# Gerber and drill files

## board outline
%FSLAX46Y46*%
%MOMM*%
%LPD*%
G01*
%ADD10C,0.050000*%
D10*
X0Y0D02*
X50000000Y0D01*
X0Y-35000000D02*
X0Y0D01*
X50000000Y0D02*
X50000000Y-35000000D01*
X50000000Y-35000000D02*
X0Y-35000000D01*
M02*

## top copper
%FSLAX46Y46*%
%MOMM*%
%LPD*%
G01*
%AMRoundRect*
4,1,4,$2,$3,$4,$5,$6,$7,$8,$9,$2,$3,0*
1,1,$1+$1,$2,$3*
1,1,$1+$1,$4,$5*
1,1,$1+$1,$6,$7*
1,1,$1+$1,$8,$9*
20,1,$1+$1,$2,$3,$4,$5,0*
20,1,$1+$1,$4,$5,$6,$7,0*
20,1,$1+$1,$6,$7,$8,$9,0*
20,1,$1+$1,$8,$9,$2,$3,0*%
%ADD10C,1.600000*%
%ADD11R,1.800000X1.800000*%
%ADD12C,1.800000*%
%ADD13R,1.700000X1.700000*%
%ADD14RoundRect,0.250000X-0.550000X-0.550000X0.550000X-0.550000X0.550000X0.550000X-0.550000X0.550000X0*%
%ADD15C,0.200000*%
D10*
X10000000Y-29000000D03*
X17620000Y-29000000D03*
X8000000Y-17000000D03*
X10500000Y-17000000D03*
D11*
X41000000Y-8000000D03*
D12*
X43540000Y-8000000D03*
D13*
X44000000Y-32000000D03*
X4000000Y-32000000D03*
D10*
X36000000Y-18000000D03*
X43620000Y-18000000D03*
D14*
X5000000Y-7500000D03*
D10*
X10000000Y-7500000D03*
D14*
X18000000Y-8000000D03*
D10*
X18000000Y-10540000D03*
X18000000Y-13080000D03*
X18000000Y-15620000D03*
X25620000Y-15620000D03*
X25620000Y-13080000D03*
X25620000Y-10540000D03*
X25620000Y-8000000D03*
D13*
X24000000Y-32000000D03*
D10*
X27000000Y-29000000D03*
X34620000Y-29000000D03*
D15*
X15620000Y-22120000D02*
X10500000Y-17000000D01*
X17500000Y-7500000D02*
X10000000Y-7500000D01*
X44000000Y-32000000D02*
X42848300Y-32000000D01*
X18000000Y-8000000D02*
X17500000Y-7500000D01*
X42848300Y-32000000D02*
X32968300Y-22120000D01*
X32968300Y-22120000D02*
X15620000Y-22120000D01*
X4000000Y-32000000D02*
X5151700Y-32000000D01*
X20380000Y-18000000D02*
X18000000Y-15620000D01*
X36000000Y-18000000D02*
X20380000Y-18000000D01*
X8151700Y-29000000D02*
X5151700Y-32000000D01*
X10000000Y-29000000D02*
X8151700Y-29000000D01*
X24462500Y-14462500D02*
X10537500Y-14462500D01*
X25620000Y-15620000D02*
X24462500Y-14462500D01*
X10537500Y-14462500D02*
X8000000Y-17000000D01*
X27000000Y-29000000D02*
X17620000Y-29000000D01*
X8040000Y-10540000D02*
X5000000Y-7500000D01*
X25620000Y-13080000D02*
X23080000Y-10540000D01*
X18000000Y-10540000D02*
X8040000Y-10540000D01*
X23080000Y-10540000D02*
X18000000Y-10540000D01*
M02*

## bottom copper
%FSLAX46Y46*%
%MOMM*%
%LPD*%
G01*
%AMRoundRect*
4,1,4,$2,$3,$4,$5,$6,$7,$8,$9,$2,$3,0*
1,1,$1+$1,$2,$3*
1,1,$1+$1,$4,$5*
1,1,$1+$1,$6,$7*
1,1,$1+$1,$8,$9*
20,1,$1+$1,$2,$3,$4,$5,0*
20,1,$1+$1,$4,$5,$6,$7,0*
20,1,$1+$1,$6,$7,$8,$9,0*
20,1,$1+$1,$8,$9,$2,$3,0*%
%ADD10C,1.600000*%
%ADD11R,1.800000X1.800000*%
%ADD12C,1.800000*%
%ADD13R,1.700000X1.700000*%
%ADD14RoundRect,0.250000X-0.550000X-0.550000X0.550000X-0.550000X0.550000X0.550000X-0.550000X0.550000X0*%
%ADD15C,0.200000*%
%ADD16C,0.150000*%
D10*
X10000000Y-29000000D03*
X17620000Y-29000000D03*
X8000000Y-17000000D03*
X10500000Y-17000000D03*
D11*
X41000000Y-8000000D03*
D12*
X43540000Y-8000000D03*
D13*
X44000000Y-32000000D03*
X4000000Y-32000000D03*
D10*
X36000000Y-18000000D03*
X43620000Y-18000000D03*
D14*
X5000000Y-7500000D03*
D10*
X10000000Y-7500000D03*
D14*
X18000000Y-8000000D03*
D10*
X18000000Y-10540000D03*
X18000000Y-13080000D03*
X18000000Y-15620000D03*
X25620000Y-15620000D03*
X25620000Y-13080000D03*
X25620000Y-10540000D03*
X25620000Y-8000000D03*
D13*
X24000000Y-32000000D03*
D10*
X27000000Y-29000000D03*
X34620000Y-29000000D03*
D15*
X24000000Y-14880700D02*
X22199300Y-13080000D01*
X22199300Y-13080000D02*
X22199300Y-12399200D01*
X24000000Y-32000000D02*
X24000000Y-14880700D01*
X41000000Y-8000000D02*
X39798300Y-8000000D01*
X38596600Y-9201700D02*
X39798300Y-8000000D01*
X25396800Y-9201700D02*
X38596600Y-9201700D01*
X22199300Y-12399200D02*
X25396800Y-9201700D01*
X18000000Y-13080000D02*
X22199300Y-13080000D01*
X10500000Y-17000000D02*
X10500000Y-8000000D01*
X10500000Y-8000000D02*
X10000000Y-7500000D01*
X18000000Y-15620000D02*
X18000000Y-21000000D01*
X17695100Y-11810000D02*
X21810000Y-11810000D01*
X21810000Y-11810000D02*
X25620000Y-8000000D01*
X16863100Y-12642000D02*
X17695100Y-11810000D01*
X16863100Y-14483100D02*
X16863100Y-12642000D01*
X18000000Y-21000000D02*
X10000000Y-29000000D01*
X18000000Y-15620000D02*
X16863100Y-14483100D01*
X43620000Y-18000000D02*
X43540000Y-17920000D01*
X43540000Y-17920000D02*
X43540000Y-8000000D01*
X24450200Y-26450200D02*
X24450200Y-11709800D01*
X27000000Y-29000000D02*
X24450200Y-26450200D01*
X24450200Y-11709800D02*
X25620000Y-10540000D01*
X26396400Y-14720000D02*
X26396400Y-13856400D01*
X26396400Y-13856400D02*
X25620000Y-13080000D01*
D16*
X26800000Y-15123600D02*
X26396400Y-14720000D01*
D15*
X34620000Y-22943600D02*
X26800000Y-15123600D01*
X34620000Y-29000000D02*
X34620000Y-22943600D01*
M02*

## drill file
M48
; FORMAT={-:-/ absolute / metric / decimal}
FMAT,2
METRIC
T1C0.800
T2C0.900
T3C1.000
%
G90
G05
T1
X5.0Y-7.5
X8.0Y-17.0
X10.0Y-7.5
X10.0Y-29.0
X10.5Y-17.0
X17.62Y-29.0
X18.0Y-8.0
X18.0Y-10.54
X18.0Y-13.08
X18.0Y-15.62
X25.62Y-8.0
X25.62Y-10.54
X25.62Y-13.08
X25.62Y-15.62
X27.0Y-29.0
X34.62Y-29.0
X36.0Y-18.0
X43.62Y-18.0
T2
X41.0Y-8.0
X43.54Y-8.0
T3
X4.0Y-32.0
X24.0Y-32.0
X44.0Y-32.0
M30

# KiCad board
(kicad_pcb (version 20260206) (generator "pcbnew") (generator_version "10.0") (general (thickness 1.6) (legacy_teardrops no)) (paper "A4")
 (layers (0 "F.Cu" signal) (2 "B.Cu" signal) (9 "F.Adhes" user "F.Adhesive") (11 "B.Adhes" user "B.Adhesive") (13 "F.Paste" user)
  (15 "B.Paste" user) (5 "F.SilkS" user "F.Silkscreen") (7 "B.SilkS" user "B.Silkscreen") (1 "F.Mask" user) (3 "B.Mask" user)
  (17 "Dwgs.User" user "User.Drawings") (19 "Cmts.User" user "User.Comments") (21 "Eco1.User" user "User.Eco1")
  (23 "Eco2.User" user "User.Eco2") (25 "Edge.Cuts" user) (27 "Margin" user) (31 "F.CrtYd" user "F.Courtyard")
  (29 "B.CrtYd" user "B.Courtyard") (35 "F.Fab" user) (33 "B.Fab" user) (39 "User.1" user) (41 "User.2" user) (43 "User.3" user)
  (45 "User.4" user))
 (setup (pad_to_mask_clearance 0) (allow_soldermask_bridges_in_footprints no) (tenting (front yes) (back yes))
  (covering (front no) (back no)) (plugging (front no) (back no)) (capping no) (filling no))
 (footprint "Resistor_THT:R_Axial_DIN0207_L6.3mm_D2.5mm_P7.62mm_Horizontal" (layer "F.Cu") (at 10 29)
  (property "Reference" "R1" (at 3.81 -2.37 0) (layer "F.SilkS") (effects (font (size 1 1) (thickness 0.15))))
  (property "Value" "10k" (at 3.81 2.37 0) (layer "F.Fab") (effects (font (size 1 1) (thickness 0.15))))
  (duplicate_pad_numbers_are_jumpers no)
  (pad "1" thru_hole circle (at 0 0) (size 1.6 1.6) (drill 0.8) (layers "*.Cu" "*.Mask") (remove_unused_layers no) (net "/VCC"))
  (pad "2" thru_hole circle (at 7.62 0) (size 1.6 1.6) (drill 0.8) (layers "*.Cu" "*.Mask") (remove_unused_layers no) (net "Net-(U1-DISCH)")))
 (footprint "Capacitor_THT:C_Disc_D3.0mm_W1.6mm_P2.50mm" (layer "F.Cu") (at 8 17)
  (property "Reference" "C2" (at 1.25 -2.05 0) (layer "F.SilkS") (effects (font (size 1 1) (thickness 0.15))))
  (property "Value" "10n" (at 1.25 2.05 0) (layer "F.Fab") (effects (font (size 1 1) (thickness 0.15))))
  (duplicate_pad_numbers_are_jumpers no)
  (pad "1" thru_hole circle (at 0 0) (size 1.6 1.6) (drill 0.8) (layers "*.Cu" "*.Mask") (remove_unused_layers no) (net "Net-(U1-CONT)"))
  (pad "2" thru_hole circle (at 2.5 0) (size 1.6 1.6) (drill 0.8) (layers "*.Cu" "*.Mask") (remove_unused_layers no) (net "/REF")))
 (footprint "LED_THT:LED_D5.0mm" (layer "F.Cu") (at 41 8)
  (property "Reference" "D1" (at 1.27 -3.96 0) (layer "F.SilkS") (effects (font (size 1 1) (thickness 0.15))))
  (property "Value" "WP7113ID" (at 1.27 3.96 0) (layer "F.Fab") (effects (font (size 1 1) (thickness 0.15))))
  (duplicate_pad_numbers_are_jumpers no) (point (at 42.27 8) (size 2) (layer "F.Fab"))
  (pad "1" thru_hole rect (at 0 0) (size 1.8 1.8) (drill 0.9) (layers "*.Cu" "*.Mask") (remove_unused_layers no) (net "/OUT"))
  (pad "2" thru_hole circle (at 2.54 0) (size 1.8 1.8) (drill 0.9) (layers "*.Cu" "*.Mask") (remove_unused_layers no) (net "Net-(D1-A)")))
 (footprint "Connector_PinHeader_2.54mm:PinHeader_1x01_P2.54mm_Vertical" (layer "F.Cu") (at 44 32)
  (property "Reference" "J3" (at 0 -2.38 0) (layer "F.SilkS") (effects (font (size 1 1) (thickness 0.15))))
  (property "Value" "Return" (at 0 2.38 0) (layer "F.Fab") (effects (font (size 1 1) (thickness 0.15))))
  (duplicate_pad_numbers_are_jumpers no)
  (pad "1" thru_hole rect (at 0 0) (size 1.7 1.7) (drill 1) (layers "*.Cu" "*.Mask") (remove_unused_layers no) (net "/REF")))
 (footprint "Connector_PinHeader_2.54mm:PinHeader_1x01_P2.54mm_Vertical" (layer "F.Cu") (at 4 32)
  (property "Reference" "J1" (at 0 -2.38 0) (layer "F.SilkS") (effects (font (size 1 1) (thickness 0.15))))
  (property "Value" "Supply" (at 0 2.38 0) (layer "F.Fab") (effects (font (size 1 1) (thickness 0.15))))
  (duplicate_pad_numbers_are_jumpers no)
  (pad "1" thru_hole rect (at 0 0) (size 1.7 1.7) (drill 1) (layers "*.Cu" "*.Mask") (remove_unused_layers no) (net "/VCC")))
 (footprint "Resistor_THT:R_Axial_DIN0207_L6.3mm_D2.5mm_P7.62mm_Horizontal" (layer "F.Cu") (at 36 18)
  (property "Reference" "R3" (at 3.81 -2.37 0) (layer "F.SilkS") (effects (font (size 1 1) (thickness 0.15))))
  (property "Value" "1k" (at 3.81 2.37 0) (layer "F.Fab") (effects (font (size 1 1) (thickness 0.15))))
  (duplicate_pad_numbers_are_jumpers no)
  (pad "1" thru_hole circle (at 0 0) (size 1.6 1.6) (drill 0.8) (layers "*.Cu" "*.Mask") (remove_unused_layers no) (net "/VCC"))
  (pad "2" thru_hole circle (at 7.62 0) (size 1.6 1.6) (drill 0.8) (layers "*.Cu" "*.Mask") (remove_unused_layers no) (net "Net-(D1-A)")))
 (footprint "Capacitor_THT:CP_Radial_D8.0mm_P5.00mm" (layer "F.Cu") (at 5 7.5)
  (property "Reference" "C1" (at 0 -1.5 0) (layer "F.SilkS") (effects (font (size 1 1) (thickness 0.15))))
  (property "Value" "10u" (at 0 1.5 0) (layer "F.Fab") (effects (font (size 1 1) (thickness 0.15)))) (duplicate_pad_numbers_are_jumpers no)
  (pad "1" thru_hole roundrect (at 0 0) (size 1.6 1.6) (drill 0.8) (layers "*.Cu" "*.Mask") (remove_unused_layers no)
   (roundrect_rratio 0.15625) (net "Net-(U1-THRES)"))
  (pad "2" thru_hole circle (at 5 0) (size 1.6 1.6) (drill 0.8) (layers "*.Cu" "*.Mask") (remove_unused_layers no) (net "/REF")))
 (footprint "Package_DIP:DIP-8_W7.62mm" (layer "F.Cu") (at 18 8)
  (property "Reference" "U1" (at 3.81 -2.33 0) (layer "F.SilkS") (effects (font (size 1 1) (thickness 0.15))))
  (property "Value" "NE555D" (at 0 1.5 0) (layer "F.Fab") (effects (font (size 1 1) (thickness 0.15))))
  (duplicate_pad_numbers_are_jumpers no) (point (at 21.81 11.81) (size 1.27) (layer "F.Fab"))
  (pad "1" thru_hole roundrect (at 0 0) (size 1.6 1.6) (drill 0.8) (layers "*.Cu" "*.Mask") (remove_unused_layers no)
   (roundrect_rratio 0.15625) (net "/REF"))
  (pad "2" thru_hole circle (at 0 2.54) (size 1.6 1.6) (drill 0.8) (layers "*.Cu" "*.Mask") (remove_unused_layers no) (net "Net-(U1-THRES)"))
  (pad "3" thru_hole circle (at 0 5.08) (size 1.6 1.6) (drill 0.8) (layers "*.Cu" "*.Mask") (remove_unused_layers no) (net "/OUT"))
  (pad "4" thru_hole circle (at 0 7.62) (size 1.6 1.6) (drill 0.8) (layers "*.Cu" "*.Mask") (remove_unused_layers no) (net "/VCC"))
  (pad "5" thru_hole circle (at 7.62 7.62) (size 1.6 1.6) (drill 0.8) (layers "*.Cu" "*.Mask") (remove_unused_layers no)
   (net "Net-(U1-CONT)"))
  (pad "6" thru_hole circle (at 7.62 5.08) (size 1.6 1.6) (drill 0.8) (layers "*.Cu" "*.Mask") (remove_unused_layers no)
   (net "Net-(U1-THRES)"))
  (pad "7" thru_hole circle (at 7.62 2.54) (size 1.6 1.6) (drill 0.8) (layers "*.Cu" "*.Mask") (remove_unused_layers no)
   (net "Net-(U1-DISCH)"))
  (pad "8" thru_hole circle (at 7.62 0) (size 1.6 1.6) (drill 0.8) (layers "*.Cu" "*.Mask") (remove_unused_layers no) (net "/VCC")))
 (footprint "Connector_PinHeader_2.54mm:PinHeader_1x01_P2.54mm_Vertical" (layer "F.Cu") (at 24 32)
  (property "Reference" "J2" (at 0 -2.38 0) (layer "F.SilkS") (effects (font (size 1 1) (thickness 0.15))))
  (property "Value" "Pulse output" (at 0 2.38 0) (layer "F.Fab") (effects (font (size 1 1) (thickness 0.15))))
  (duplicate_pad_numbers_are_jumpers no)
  (pad "1" thru_hole rect (at 0 0) (size 1.7 1.7) (drill 1) (layers "*.Cu" "*.Mask") (remove_unused_layers no) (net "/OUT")))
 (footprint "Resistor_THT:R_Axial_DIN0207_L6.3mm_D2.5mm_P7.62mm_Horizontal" (layer "F.Cu") (at 27 29)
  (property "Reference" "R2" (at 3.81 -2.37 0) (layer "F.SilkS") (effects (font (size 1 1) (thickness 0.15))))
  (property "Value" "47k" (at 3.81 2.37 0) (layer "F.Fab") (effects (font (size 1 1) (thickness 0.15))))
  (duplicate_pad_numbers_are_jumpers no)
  (pad "1" thru_hole circle (at 0 0) (size 1.6 1.6) (drill 0.8) (layers "*.Cu" "*.Mask") (remove_unused_layers no) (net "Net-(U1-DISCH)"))
  (pad "2" thru_hole circle (at 7.62 0) (size 1.6 1.6) (drill 0.8) (layers "*.Cu" "*.Mask") (remove_unused_layers no) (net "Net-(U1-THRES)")))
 (gr_line (start 0 0) (end 50 0) (stroke (width 0.05) (type default)) (layer "Edge.Cuts"))
 (gr_line (start 0 35) (end 0 0) (stroke (width 0.05) (type default)) (layer "Edge.Cuts"))
 (gr_line (start 50 0) (end 50 35) (stroke (width 0.05) (type default)) (layer "Edge.Cuts"))
 (gr_line (start 50 35) (end 0 35) (stroke (width 0.05) (type default)) (layer "Edge.Cuts"))
 (segment (start 24 14.8807) (end 22.1993 13.08) (width 0.2) (layer "B.Cu") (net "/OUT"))
 (segment (start 22.1993 13.08) (end 22.1993 12.3992) (width 0.2) (layer "B.Cu") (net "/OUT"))
 (segment (start 24 32) (end 24 14.8807) (width 0.2) (layer "B.Cu") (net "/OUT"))
 (segment (start 41 8) (end 39.7983 8) (width 0.2) (layer "B.Cu") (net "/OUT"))
 (segment (start 38.5966 9.2017) (end 39.7983 8) (width 0.2) (layer "B.Cu") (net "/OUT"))
 (segment (start 25.3968 9.2017) (end 38.5966 9.2017) (width 0.2) (layer "B.Cu") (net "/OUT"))
 (segment (start 22.1993 12.3992) (end 25.3968 9.2017) (width 0.2) (layer "B.Cu") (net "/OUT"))
 (segment (start 18 13.08) (end 22.1993 13.08) (width 0.2) (layer "B.Cu") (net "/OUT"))
 (segment (start 15.62 22.12) (end 10.5 17) (width 0.2) (layer "F.Cu") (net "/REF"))
 (segment (start 17.5 7.5) (end 10 7.5) (width 0.2) (layer "F.Cu") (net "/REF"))
 (segment (start 44 32) (end 42.8483 32) (width 0.2) (layer "F.Cu") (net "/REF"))
 (segment (start 18 8) (end 17.5 7.5) (width 0.2) (layer "F.Cu") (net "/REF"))
 (segment (start 42.8483 32) (end 32.9683 22.12) (width 0.2) (layer "F.Cu") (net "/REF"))
 (segment (start 32.9683 22.12) (end 15.62 22.12) (width 0.2) (layer "F.Cu") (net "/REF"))
 (segment (start 10.5 17) (end 10.5 8) (width 0.2) (layer "B.Cu") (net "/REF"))
 (segment (start 10.5 8) (end 10 7.5) (width 0.2) (layer "B.Cu") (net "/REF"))
 (segment (start 4 32) (end 5.1517 32) (width 0.2) (layer "F.Cu") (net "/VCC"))
 (segment (start 20.38 18) (end 18 15.62) (width 0.2) (layer "F.Cu") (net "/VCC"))
 (segment (start 36 18) (end 20.38 18) (width 0.2) (layer "F.Cu") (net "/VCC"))
 (segment (start 8.1517 29) (end 5.1517 32) (width 0.2) (layer "F.Cu") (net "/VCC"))
 (segment (start 10 29) (end 8.1517 29) (width 0.2) (layer "F.Cu") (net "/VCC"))
 (segment (start 18 15.62) (end 18 21) (width 0.2) (layer "B.Cu") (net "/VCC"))
 (segment (start 17.6951 11.81) (end 21.81 11.81) (width 0.2) (layer "B.Cu") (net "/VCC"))
 (segment (start 21.81 11.81) (end 25.62 8) (width 0.2) (layer "B.Cu") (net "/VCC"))
 (segment (start 16.8631 12.642) (end 17.6951 11.81) (width 0.2) (layer "B.Cu") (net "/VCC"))
 (segment (start 16.8631 14.4831) (end 16.8631 12.642) (width 0.2) (layer "B.Cu") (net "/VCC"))
 (segment (start 18 21) (end 10 29) (width 0.2) (layer "B.Cu") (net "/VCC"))
 (segment (start 18 15.62) (end 16.8631 14.4831) (width 0.2) (layer "B.Cu") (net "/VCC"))
 (segment (start 43.62 18) (end 43.54 17.92) (width 0.2) (layer "B.Cu") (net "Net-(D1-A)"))
 (segment (start 43.54 17.92) (end 43.54 8) (width 0.2) (layer "B.Cu") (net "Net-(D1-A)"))
 (segment (start 24.4625 14.4625) (end 10.5375 14.4625) (width 0.2) (layer "F.Cu") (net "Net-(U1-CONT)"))
 (segment (start 25.62 15.62) (end 24.4625 14.4625) (width 0.2) (layer "F.Cu") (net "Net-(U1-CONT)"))
 (segment (start 10.5375 14.4625) (end 8 17) (width 0.2) (layer "F.Cu") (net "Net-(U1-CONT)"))
 (segment (start 27 29) (end 17.62 29) (width 0.2) (layer "F.Cu") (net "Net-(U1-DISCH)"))
 (segment (start 24.4502 26.4502) (end 24.4502 11.7098) (width 0.2) (layer "B.Cu") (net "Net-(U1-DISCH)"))
 (segment (start 27 29) (end 24.4502 26.4502) (width 0.2) (layer "B.Cu") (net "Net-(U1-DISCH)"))
 (segment (start 24.4502 11.7098) (end 25.62 10.54) (width 0.2) (layer "B.Cu") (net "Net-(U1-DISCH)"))
 (segment (start 8.04 10.54) (end 5 7.5) (width 0.2) (layer "F.Cu") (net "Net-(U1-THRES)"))
 (segment (start 25.62 13.08) (end 23.08 10.54) (width 0.2) (layer "F.Cu") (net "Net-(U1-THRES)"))
 (segment (start 18 10.54) (end 8.04 10.54) (width 0.2) (layer "F.Cu") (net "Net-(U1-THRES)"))
 (segment (start 23.08 10.54) (end 18 10.54) (width 0.2) (layer "F.Cu") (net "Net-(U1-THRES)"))
 (segment (start 26.3964 14.72) (end 26.3964 13.8564) (width 0.2) (layer "B.Cu") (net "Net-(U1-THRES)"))
 (segment (start 26.3964 13.8564) (end 25.62 13.08) (width 0.2) (layer "B.Cu") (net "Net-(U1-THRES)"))
 (segment (start 26.8 15.1236) (end 26.3964 14.72) (width 0.15) (layer "B.Cu") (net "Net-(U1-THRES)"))
 (segment (start 34.62 22.9436) (end 26.8 15.1236) (width 0.2) (layer "B.Cu") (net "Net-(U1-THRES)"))
 (segment (start 34.62 29) (end 34.62 22.9436) (width 0.2) (layer "B.Cu") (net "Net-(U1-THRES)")))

